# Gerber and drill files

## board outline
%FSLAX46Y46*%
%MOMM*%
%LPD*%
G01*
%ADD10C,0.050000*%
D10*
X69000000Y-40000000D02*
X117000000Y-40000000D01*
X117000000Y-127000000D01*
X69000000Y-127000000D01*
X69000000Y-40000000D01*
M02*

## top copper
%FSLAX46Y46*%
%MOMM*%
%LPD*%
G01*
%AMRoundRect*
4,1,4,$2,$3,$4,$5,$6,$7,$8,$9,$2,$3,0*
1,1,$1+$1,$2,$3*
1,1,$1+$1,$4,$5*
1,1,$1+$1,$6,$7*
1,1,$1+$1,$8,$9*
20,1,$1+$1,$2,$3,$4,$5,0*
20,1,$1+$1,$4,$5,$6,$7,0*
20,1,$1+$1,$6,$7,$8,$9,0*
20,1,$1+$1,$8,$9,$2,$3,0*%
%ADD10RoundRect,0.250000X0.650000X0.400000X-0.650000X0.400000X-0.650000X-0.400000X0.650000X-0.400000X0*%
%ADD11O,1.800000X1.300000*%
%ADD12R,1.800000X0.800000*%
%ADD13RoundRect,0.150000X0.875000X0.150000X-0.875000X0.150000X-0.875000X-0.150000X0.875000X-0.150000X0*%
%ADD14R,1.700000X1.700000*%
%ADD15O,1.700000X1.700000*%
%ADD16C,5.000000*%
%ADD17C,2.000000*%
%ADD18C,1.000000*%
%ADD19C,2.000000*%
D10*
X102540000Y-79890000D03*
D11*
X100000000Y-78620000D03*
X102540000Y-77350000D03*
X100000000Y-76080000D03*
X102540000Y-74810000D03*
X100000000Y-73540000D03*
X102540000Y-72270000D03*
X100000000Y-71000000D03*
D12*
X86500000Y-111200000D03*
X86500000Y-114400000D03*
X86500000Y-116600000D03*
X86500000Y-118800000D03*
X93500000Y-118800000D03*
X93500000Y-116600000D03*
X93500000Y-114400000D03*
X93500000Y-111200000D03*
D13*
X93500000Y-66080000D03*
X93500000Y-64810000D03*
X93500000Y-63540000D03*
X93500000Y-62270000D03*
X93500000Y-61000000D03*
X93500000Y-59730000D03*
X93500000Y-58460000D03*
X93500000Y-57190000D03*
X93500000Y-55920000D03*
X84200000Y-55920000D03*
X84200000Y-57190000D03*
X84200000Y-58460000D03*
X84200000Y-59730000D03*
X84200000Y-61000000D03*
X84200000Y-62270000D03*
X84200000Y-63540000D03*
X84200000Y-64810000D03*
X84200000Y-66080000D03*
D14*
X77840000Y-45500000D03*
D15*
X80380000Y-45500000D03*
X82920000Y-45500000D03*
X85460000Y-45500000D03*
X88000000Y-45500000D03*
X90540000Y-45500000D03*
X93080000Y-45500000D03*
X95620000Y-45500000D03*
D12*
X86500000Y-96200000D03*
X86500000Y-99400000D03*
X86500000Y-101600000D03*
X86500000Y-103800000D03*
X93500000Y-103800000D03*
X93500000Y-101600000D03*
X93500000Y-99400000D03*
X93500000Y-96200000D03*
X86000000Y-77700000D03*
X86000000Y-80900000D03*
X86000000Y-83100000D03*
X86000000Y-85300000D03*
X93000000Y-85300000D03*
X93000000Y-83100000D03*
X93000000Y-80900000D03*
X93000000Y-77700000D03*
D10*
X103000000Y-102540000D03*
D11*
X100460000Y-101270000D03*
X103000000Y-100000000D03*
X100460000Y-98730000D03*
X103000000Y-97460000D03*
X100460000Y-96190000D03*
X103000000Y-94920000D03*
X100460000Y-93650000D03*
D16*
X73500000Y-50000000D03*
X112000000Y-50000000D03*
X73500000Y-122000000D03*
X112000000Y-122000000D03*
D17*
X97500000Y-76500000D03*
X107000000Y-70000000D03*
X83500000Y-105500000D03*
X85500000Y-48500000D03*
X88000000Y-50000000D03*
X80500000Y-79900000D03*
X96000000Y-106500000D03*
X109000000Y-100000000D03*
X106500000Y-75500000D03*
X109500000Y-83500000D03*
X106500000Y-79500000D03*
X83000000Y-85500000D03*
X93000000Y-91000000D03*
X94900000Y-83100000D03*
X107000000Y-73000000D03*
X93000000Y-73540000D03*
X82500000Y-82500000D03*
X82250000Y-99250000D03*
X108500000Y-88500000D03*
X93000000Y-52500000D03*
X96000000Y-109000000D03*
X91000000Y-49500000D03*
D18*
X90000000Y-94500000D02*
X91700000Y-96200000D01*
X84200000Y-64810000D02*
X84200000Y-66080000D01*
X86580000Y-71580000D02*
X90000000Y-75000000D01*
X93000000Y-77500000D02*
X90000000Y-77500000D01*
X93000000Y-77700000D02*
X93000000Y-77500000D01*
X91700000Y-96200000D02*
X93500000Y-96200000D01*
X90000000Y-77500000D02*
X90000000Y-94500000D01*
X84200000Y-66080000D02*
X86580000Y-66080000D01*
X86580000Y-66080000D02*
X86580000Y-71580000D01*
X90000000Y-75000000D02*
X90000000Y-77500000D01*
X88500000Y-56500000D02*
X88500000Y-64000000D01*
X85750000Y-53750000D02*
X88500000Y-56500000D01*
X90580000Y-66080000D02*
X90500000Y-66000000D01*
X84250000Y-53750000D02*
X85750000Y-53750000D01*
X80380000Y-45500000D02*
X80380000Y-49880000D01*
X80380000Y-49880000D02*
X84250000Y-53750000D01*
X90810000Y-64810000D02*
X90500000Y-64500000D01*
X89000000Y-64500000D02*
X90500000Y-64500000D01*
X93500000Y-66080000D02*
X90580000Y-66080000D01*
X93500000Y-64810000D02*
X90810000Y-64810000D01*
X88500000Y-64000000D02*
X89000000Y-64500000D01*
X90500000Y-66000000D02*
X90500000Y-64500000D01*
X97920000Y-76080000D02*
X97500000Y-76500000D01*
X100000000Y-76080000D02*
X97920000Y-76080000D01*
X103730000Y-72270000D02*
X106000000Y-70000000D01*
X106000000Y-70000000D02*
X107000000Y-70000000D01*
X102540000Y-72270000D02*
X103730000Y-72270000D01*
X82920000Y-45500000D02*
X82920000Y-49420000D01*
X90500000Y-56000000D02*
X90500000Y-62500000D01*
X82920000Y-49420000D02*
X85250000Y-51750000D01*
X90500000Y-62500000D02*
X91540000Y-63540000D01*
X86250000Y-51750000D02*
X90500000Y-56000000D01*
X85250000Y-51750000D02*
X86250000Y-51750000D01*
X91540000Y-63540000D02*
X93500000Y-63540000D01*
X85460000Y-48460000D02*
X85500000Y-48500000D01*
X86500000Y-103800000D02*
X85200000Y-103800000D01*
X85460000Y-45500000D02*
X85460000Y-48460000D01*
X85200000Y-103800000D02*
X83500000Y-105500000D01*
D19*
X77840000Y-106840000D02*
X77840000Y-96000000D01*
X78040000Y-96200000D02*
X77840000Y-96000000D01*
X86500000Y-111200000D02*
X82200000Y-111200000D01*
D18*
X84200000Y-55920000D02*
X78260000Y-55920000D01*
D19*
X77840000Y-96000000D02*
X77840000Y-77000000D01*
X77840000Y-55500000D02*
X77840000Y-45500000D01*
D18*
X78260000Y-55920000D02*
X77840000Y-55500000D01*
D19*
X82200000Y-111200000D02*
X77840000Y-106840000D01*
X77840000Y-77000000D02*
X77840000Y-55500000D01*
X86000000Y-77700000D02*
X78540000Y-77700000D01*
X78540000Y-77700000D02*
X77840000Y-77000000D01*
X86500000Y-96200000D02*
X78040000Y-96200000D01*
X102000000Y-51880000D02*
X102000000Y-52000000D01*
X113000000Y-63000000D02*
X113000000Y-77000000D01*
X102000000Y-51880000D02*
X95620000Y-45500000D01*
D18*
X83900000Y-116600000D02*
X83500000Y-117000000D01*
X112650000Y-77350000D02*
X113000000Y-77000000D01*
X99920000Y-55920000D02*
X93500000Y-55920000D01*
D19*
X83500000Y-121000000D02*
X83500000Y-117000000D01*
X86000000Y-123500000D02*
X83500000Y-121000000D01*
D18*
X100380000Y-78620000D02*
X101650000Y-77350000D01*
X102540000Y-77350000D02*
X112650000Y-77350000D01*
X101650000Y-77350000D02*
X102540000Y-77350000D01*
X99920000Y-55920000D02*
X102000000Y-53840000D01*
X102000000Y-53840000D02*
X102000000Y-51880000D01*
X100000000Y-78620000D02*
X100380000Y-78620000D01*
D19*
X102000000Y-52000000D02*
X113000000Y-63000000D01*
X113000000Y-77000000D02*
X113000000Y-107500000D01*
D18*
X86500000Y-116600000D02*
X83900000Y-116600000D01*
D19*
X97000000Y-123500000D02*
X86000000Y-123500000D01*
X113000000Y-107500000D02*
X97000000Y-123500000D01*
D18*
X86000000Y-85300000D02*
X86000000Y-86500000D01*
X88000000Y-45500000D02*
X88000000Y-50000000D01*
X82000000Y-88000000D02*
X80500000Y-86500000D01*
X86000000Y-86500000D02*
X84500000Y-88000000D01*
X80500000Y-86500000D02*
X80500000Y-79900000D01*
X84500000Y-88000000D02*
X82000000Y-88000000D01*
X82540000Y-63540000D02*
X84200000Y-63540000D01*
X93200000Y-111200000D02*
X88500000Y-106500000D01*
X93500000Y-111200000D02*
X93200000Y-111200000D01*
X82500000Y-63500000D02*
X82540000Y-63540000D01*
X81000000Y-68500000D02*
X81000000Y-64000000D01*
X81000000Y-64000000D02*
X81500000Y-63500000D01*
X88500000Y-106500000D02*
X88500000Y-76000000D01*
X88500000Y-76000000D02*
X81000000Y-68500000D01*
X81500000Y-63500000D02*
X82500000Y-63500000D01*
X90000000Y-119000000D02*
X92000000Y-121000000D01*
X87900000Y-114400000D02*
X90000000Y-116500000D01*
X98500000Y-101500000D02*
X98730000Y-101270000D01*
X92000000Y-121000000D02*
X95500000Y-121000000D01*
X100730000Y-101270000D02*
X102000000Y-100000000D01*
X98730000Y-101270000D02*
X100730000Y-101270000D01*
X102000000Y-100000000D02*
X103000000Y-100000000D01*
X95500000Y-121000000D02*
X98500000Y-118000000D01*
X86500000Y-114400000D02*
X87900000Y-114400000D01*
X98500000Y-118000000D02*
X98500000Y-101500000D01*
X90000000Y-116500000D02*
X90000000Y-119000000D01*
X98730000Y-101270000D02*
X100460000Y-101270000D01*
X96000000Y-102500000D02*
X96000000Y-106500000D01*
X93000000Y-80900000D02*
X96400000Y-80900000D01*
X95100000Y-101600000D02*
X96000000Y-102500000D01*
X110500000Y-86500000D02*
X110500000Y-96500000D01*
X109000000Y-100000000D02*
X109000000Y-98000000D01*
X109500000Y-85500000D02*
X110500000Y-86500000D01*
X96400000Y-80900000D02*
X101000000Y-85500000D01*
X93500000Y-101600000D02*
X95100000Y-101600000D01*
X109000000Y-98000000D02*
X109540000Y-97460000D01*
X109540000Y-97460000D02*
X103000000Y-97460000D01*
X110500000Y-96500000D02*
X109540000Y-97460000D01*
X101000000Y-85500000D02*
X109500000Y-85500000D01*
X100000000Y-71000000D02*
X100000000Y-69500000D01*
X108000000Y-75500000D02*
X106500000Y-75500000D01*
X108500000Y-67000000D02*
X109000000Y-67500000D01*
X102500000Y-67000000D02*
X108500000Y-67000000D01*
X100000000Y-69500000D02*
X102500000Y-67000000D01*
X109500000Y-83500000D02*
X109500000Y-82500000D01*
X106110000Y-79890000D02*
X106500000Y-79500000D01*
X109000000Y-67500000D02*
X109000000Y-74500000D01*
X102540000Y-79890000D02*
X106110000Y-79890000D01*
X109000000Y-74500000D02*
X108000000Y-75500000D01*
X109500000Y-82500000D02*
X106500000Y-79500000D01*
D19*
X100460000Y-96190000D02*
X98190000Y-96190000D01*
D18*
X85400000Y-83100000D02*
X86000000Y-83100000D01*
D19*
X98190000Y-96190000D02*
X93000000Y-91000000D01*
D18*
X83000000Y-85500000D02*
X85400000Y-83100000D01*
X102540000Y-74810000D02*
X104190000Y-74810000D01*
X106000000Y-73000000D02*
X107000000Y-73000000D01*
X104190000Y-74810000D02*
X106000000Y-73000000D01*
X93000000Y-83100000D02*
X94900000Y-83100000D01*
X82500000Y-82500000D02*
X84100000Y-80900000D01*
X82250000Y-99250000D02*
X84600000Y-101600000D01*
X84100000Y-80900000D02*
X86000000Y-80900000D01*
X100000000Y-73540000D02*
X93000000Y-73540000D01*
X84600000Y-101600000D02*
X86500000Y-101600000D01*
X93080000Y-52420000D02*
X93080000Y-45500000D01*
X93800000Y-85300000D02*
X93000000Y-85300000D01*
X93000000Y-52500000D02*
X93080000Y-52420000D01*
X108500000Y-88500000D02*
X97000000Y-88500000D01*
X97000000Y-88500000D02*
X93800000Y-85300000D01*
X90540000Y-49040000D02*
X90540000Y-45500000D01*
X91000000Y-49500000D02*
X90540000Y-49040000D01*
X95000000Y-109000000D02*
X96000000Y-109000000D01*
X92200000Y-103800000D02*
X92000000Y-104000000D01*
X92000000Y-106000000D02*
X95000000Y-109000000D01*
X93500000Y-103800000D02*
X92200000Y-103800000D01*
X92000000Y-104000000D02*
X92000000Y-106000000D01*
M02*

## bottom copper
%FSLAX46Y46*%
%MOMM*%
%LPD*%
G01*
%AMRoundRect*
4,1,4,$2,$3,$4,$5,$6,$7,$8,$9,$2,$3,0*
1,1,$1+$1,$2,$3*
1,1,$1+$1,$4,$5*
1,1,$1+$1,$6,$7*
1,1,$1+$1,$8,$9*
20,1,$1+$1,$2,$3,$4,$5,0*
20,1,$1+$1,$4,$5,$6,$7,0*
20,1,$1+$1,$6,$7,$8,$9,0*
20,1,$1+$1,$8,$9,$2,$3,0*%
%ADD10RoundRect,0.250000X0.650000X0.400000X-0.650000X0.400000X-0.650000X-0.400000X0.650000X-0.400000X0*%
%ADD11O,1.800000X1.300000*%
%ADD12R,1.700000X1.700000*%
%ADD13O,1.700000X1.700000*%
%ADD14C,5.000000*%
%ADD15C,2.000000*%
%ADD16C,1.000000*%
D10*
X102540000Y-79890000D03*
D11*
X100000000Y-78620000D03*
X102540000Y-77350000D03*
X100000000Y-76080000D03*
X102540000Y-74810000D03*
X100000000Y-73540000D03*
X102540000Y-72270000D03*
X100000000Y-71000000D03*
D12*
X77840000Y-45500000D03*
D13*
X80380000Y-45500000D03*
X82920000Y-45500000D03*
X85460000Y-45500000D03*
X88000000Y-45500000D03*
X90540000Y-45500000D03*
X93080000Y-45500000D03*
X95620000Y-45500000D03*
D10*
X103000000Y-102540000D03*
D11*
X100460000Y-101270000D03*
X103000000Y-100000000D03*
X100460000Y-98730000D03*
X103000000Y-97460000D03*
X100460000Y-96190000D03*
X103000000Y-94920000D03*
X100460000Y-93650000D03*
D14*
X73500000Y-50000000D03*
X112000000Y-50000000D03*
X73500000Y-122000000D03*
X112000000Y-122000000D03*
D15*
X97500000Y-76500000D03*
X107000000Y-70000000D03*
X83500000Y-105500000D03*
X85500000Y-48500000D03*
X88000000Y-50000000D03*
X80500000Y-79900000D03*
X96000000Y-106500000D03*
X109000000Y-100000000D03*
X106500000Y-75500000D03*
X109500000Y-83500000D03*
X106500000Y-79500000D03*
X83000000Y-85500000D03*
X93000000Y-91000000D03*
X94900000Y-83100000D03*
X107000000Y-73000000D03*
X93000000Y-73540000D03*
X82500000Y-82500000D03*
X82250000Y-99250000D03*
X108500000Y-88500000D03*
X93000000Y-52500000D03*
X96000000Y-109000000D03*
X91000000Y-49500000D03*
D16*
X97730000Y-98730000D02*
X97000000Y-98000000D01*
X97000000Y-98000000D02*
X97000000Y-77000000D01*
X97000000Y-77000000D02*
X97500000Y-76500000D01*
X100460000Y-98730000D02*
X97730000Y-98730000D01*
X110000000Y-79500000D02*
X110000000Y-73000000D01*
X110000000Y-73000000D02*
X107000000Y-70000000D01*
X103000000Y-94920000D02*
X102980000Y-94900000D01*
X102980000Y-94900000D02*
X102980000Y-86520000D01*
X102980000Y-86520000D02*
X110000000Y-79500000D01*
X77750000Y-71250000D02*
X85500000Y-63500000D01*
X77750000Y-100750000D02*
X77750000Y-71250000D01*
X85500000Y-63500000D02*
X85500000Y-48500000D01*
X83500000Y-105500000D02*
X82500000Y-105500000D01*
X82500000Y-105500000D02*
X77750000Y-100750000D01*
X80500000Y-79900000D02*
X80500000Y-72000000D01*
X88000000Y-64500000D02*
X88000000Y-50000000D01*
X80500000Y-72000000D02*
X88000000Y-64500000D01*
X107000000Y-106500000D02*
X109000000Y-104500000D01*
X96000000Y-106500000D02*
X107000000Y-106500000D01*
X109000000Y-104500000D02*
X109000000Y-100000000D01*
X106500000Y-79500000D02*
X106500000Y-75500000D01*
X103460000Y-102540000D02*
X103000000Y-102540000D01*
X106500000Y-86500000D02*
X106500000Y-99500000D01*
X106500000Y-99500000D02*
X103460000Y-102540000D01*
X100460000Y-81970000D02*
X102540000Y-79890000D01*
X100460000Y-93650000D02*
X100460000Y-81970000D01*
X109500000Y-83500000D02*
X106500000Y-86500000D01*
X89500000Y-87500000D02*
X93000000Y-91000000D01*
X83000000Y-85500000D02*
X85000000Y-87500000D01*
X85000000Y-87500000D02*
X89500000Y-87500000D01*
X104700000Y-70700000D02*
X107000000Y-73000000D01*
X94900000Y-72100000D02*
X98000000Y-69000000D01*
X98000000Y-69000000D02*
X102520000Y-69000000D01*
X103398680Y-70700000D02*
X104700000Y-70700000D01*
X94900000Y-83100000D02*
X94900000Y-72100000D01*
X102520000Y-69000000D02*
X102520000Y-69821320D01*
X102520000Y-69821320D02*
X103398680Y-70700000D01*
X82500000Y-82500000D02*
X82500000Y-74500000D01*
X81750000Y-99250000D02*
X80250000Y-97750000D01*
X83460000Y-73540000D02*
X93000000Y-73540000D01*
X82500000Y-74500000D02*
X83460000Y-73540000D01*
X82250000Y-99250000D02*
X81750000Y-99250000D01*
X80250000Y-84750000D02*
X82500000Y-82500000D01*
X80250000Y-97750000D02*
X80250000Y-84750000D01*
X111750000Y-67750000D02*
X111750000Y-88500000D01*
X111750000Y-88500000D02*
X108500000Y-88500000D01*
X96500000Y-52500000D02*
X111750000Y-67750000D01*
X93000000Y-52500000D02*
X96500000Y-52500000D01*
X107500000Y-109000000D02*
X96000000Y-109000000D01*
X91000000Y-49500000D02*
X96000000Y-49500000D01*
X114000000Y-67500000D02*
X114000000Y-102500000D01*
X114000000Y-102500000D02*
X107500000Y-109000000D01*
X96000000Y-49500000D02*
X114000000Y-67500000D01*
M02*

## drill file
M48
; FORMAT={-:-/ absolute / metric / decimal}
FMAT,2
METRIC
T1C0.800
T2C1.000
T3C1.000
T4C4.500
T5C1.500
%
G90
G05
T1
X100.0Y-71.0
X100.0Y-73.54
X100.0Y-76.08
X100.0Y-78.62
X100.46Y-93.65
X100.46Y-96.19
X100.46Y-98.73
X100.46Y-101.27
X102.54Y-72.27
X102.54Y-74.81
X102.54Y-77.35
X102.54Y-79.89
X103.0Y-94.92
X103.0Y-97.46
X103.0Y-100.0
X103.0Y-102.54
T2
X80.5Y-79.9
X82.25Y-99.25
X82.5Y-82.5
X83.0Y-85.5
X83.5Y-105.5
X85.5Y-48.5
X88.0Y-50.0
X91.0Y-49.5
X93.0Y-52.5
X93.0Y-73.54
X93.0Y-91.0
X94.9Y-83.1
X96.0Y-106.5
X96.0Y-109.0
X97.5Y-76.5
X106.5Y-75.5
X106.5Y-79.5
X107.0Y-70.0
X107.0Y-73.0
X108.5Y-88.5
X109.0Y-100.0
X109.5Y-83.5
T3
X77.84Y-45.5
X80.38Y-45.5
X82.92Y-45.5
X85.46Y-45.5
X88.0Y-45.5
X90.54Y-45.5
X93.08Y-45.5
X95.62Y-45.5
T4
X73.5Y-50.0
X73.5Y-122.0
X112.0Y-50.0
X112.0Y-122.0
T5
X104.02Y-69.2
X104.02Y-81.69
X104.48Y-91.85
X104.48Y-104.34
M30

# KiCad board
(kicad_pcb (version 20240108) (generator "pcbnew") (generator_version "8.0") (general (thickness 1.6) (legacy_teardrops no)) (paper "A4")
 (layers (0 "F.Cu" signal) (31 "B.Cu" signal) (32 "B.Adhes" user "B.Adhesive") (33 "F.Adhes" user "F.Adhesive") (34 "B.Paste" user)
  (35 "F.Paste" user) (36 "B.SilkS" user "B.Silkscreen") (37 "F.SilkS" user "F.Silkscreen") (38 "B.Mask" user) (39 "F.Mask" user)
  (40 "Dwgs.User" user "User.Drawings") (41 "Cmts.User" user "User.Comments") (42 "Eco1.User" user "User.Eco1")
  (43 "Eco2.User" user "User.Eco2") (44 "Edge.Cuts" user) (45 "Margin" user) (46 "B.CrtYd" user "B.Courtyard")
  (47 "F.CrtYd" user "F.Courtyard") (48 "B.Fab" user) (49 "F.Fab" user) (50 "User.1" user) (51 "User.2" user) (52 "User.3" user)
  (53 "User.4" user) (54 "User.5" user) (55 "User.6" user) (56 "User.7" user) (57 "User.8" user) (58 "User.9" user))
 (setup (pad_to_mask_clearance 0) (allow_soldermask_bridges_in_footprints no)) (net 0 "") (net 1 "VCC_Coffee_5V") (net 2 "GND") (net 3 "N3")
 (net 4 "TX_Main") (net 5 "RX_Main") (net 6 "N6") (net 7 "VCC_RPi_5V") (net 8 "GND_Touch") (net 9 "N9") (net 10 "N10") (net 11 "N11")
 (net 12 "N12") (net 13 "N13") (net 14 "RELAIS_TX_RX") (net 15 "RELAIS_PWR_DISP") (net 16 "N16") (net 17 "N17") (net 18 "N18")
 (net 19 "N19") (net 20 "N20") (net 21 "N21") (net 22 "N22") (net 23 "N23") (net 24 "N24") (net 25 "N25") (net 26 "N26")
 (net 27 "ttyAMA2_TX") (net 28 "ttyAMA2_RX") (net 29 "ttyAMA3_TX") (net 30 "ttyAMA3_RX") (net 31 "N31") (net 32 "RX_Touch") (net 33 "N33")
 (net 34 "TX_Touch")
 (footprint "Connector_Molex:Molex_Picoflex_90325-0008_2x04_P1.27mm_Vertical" (layer "F.Cu") (at 102.54 79.89 180)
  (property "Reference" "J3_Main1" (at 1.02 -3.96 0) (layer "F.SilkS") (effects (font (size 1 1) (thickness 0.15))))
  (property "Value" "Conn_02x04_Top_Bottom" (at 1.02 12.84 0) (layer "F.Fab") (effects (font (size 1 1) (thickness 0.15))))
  (pad "" np_thru_hole circle (at -1.48 -1.8 180) (size 1.5 1.5) (drill 1.5) (layers "*.Cu" "*.Mask"))
  (pad "" np_thru_hole circle (at -1.48 10.69 180) (size 1.5 1.5) (drill 1.5) (layers "*.Cu" "*.Mask"))
  (pad "1" thru_hole roundrect (at 0 0 180) (size 1.8 1.3) (drill 0.8) (layers "*.Cu" "*.Mask") (remove_unused_layers no)
   (roundrect_rratio 0.192308) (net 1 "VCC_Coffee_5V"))
  (pad "2" thru_hole oval (at 2.54 1.27 180) (size 1.8 1.3) (drill 0.8) (layers "*.Cu" "*.Mask") (remove_unused_layers no) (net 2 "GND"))
  (pad "3" thru_hole oval (at 0 2.54 180) (size 1.8 1.3) (drill 0.8) (layers "*.Cu" "*.Mask") (remove_unused_layers no) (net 2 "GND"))
  (pad "4" thru_hole oval (at 2.54 3.81 180) (size 1.8 1.3) (drill 0.8) (layers "*.Cu" "*.Mask") (remove_unused_layers no) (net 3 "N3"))
  (pad "5" thru_hole oval (at 0 5.08 180) (size 1.8 1.3) (drill 0.8) (layers "*.Cu" "*.Mask") (remove_unused_layers no) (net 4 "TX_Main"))
  (pad "6" thru_hole oval (at 2.54 6.35 180) (size 1.8 1.3) (drill 0.8) (layers "*.Cu" "*.Mask") (remove_unused_layers no) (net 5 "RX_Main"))
  (pad "7" thru_hole oval (at 0 7.62 180) (size 1.8 1.3) (drill 0.8) (layers "*.Cu" "*.Mask") (remove_unused_layers no) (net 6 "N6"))
  (pad "8" thru_hole oval (at 2.54 8.89 180) (size 1.8 1.3) (drill 0.8) (layers "*.Cu" "*.Mask") (remove_unused_layers no)
   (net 1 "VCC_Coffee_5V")))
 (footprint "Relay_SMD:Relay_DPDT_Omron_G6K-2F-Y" (layer "F.Cu") (at 90 115)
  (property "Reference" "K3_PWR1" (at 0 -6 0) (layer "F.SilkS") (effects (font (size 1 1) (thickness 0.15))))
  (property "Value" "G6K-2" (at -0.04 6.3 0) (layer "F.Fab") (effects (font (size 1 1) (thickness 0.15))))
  (pad "1" smd rect (at -3.5 -3.8) (size 1.8 0.8) (layers "F.Cu" "F.Paste" "F.Mask") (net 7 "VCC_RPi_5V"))
  (pad "2" smd rect (at -3.5 -0.6) (size 1.8 0.8) (layers "F.Cu" "F.Paste" "F.Mask") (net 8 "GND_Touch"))
  (pad "3" smd rect (at -3.5 1.6) (size 1.8 0.8) (layers "F.Cu" "F.Paste" "F.Mask") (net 2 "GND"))
  (pad "4" smd rect (at -3.5 3.8) (size 1.8 0.8) (layers "F.Cu" "F.Paste" "F.Mask") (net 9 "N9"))
  (pad "5" smd rect (at 3.5 3.8) (size 1.8 0.8) (layers "F.Cu" "F.Paste" "F.Mask") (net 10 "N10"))
  (pad "6" smd rect (at 3.5 1.6) (size 1.8 0.8) (layers "F.Cu" "F.Paste" "F.Mask") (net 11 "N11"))
  (pad "7" smd rect (at 3.5 -0.6) (size 1.8 0.8) (layers "F.Cu" "F.Paste" "F.Mask") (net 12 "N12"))
  (pad "8" smd rect (at 3.5 -3.8) (size 1.8 0.8) (layers "F.Cu" "F.Paste" "F.Mask") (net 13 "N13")))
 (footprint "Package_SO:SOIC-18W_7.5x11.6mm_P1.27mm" (layer "F.Cu") (at 88.85 61 180)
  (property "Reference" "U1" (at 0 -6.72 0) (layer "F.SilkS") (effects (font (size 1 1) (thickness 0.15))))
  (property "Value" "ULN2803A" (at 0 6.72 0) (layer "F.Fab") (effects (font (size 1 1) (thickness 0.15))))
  (pad "1" smd roundrect (at -4.65 -5.08 180) (size 2.05 0.6) (layers "F.Cu" "F.Paste" "F.Mask") (roundrect_rratio 0.25)
   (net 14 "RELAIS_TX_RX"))
  (pad "2" smd roundrect (at -4.65 -3.81 180) (size 2.05 0.6) (layers "F.Cu" "F.Paste" "F.Mask") (roundrect_rratio 0.25)
   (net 14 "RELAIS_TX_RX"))
  (pad "3" smd roundrect (at -4.65 -2.54 180) (size 2.05 0.6) (layers "F.Cu" "F.Paste" "F.Mask") (roundrect_rratio 0.25)
   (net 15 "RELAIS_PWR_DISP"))
  (pad "4" smd roundrect (at -4.65 -1.27 180) (size 2.05 0.6) (layers "F.Cu" "F.Paste" "F.Mask") (roundrect_rratio 0.25) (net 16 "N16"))
  (pad "5" smd roundrect (at -4.65 0 180) (size 2.05 0.6) (layers "F.Cu" "F.Paste" "F.Mask") (roundrect_rratio 0.25) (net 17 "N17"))
  (pad "6" smd roundrect (at -4.65 1.27 180) (size 2.05 0.6) (layers "F.Cu" "F.Paste" "F.Mask") (roundrect_rratio 0.25) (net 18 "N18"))
  (pad "7" smd roundrect (at -4.65 2.54 180) (size 2.05 0.6) (layers "F.Cu" "F.Paste" "F.Mask") (roundrect_rratio 0.25) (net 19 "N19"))
  (pad "8" smd roundrect (at -4.65 3.81 180) (size 2.05 0.6) (layers "F.Cu" "F.Paste" "F.Mask") (roundrect_rratio 0.25) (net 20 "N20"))
  (pad "9" smd roundrect (at -4.65 5.08 180) (size 2.05 0.6) (layers "F.Cu" "F.Paste" "F.Mask") (roundrect_rratio 0.25) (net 2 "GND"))
  (pad "10" smd roundrect (at 4.65 5.08 180) (size 2.05 0.6) (layers "F.Cu" "F.Paste" "F.Mask") (roundrect_rratio 0.25) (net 7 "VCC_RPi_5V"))
  (pad "11" smd roundrect (at 4.65 3.81 180) (size 2.05 0.6) (layers "F.Cu" "F.Paste" "F.Mask") (roundrect_rratio 0.25) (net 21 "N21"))
  (pad "12" smd roundrect (at 4.65 2.54 180) (size 2.05 0.6) (layers "F.Cu" "F.Paste" "F.Mask") (roundrect_rratio 0.25) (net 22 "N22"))
  (pad "13" smd roundrect (at 4.65 1.27 180) (size 2.05 0.6) (layers "F.Cu" "F.Paste" "F.Mask") (roundrect_rratio 0.25) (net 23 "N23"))
  (pad "14" smd roundrect (at 4.65 0 180) (size 2.05 0.6) (layers "F.Cu" "F.Paste" "F.Mask") (roundrect_rratio 0.25) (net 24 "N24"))
  (pad "15" smd roundrect (at 4.65 -1.27 180) (size 2.05 0.6) (layers "F.Cu" "F.Paste" "F.Mask") (roundrect_rratio 0.25) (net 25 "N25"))
  (pad "16" smd roundrect (at 4.65 -2.54 180) (size 2.05 0.6) (layers "F.Cu" "F.Paste" "F.Mask") (roundrect_rratio 0.25) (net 13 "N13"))
  (pad "17" smd roundrect (at 4.65 -3.81 180) (size 2.05 0.6) (layers "F.Cu" "F.Paste" "F.Mask") (roundrect_rratio 0.25) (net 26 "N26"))
  (pad "18" smd roundrect (at 4.65 -5.08 180) (size 2.05 0.6) (layers "F.Cu" "F.Paste" "F.Mask") (roundrect_rratio 0.25) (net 26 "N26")))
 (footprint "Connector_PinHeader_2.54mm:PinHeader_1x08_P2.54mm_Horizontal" (layer "F.Cu") (at 77.84 45.5 90)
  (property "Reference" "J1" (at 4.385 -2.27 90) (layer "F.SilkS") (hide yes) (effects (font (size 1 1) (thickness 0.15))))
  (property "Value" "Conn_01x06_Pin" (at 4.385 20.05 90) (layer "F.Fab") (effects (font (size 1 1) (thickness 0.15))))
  (pad "1" thru_hole rect (at 0 0 90) (size 1.7 1.7) (drill 1) (layers "*.Cu" "*.Mask") (remove_unused_layers no) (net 7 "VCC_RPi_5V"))
  (pad "2" thru_hole oval (at 0 2.54 90) (size 1.7 1.7) (drill 1) (layers "*.Cu" "*.Mask") (remove_unused_layers no) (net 14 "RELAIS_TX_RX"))
  (pad "3" thru_hole oval (at 0 5.08 90) (size 1.7 1.7) (drill 1) (layers "*.Cu" "*.Mask") (remove_unused_layers no)
   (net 15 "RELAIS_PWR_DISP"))
  (pad "4" thru_hole oval (at 0 7.62 90) (size 1.7 1.7) (drill 1) (layers "*.Cu" "*.Mask") (remove_unused_layers no) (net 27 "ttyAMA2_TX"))
  (pad "5" thru_hole oval (at 0 10.16 90) (size 1.7 1.7) (drill 1) (layers "*.Cu" "*.Mask") (remove_unused_layers no) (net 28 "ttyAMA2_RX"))
  (pad "6" thru_hole oval (at 0 12.7 90) (size 1.7 1.7) (drill 1) (layers "*.Cu" "*.Mask") (remove_unused_layers no) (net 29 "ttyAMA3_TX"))
  (pad "7" thru_hole oval (at 0 15.24 90) (size 1.7 1.7) (drill 1) (layers "*.Cu" "*.Mask") (remove_unused_layers no) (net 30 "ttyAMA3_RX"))
  (pad "8" thru_hole oval (at 0 17.78 90) (size 1.7 1.7) (drill 1) (layers "*.Cu" "*.Mask") (remove_unused_layers no) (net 2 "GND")))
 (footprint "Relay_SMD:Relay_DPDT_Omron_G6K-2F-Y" (layer "F.Cu") (at 90 100)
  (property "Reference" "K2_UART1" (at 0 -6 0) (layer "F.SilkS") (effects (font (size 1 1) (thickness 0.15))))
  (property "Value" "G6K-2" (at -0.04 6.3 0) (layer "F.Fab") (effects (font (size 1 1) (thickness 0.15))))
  (pad "1" smd rect (at -3.5 -3.8) (size 1.8 0.8) (layers "F.Cu" "F.Paste" "F.Mask") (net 7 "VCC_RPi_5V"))
  (pad "2" smd rect (at -3.5 -0.6) (size 1.8 0.8) (layers "F.Cu" "F.Paste" "F.Mask") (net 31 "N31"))
  (pad "3" smd rect (at -3.5 1.6) (size 1.8 0.8) (layers "F.Cu" "F.Paste" "F.Mask") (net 5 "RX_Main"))
  (pad "4" smd rect (at -3.5 3.8) (size 1.8 0.8) (layers "F.Cu" "F.Paste" "F.Mask") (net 27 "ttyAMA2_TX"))
  (pad "5" smd rect (at 3.5 3.8) (size 1.8 0.8) (layers "F.Cu" "F.Paste" "F.Mask") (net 29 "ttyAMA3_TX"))
  (pad "6" smd rect (at 3.5 1.6) (size 1.8 0.8) (layers "F.Cu" "F.Paste" "F.Mask") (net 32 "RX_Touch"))
  (pad "7" smd rect (at 3.5 -0.6) (size 1.8 0.8) (layers "F.Cu" "F.Paste" "F.Mask") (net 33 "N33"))
  (pad "8" smd rect (at 3.5 -3.8) (size 1.8 0.8) (layers "F.Cu" "F.Paste" "F.Mask") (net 26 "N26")))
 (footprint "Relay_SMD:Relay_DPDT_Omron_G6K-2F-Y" (layer "F.Cu") (at 89.5 81.5)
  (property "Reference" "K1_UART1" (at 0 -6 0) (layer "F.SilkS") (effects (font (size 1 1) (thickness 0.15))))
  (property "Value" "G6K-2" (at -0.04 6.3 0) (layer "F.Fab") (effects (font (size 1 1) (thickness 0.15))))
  (pad "1" smd rect (at -3.5 -3.8) (size 1.8 0.8) (layers "F.Cu" "F.Paste" "F.Mask") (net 7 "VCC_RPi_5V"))
  (pad "2" smd rect (at -3.5 -0.6) (size 1.8 0.8) (layers "F.Cu" "F.Paste" "F.Mask") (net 5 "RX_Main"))
  (pad "3" smd rect (at -3.5 1.6) (size 1.8 0.8) (layers "F.Cu" "F.Paste" "F.Mask") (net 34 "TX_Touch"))
  (pad "4" smd rect (at -3.5 3.8) (size 1.8 0.8) (layers "F.Cu" "F.Paste" "F.Mask") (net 28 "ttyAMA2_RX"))
  (pad "5" smd rect (at 3.5 3.8) (size 1.8 0.8) (layers "F.Cu" "F.Paste" "F.Mask") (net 30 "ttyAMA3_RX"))
  (pad "6" smd rect (at 3.5 1.6) (size 1.8 0.8) (layers "F.Cu" "F.Paste" "F.Mask") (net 4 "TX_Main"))
  (pad "7" smd rect (at 3.5 -0.6) (size 1.8 0.8) (layers "F.Cu" "F.Paste" "F.Mask") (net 32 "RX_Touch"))
  (pad "8" smd rect (at 3.5 -3.8) (size 1.8 0.8) (layers "F.Cu" "F.Paste" "F.Mask") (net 26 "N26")))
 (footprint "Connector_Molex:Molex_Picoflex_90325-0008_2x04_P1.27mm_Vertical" (layer "F.Cu") (at 103 102.54 180)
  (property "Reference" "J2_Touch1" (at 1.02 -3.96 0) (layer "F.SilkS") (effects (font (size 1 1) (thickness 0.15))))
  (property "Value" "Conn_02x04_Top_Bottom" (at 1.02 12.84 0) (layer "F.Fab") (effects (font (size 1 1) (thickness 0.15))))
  (pad "" np_thru_hole circle (at -1.48 -1.8 180) (size 1.5 1.5) (drill 1.5) (layers "*.Cu" "*.Mask"))
  (pad "" np_thru_hole circle (at -1.48 10.69 180) (size 1.5 1.5) (drill 1.5) (layers "*.Cu" "*.Mask"))
  (pad "1" thru_hole roundrect (at 0 0 180) (size 1.8 1.3) (drill 0.8) (layers "*.Cu" "*.Mask") (remove_unused_layers no)
   (roundrect_rratio 0.192308) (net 1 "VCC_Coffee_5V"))
  (pad "2" thru_hole oval (at 2.54 1.27 180) (size 1.8 1.3) (drill 0.8) (layers "*.Cu" "*.Mask") (remove_unused_layers no)
   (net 8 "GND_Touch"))
  (pad "3" thru_hole oval (at 0 2.54 180) (size 1.8 1.3) (drill 0.8) (layers "*.Cu" "*.Mask") (remove_unused_layers no) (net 8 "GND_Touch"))
  (pad "4" thru_hole oval (at 2.54 3.81 180) (size 1.8 1.3) (drill 0.8) (layers "*.Cu" "*.Mask") (remove_unused_layers no) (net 3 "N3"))
  (pad "5" thru_hole oval (at 0 5.08 180) (size 1.8 1.3) (drill 0.8) (layers "*.Cu" "*.Mask") (remove_unused_layers no) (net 32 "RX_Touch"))
  (pad "6" thru_hole oval (at 2.54 6.35 180) (size 1.8 1.3) (drill 0.8) (layers "*.Cu" "*.Mask") (remove_unused_layers no)
   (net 34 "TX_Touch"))
  (pad "7" thru_hole oval (at 0 7.62 180) (size 1.8 1.3) (drill 0.8) (layers "*.Cu" "*.Mask") (remove_unused_layers no) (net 6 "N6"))
  (pad "8" thru_hole oval (at 2.54 8.89 180) (size 1.8 1.3) (drill 0.8) (layers "*.Cu" "*.Mask") (remove_unused_layers no)
   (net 1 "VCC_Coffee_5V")))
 (gr_rect (start 69 40) (end 117 127) (stroke (width 0.05) (type default)) (fill none) (layer "Edge.Cuts"))
 (via (at 73.5 50) (size 5) (drill 4.5) (layers "F.Cu" "B.Cu") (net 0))
 (via (at 112 50) (size 5) (drill 4.5) (layers "F.Cu" "B.Cu") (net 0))
 (via (at 73.5 122) (size 5) (drill 4.5) (layers "F.Cu" "B.Cu") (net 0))
 (via (at 112 122) (size 5) (drill 4.5) (layers "F.Cu" "B.Cu") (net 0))
 (segment (start 90 94.5) (end 91.7 96.2) (width 1) (layer "F.Cu") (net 26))
 (segment (start 84.2 64.81) (end 84.2 66.08) (width 1) (layer "F.Cu") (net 26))
 (segment (start 86.58 71.58) (end 90 75) (width 1) (layer "F.Cu") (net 26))
 (segment (start 93 77.5) (end 90 77.5) (width 1) (layer "F.Cu") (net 26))
 (segment (start 93 77.7) (end 93 77.5) (width 1) (layer "F.Cu") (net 26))
 (segment (start 91.7 96.2) (end 93.5 96.2) (width 1) (layer "F.Cu") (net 26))
 (segment (start 90 77.5) (end 90 94.5) (width 1) (layer "F.Cu") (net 26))
 (segment (start 84.2 66.08) (end 86.58 66.08) (width 1) (layer "F.Cu") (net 26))
 (segment (start 86.58 66.08) (end 86.58 71.58) (width 1) (layer "F.Cu") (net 26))
 (segment (start 90 75) (end 90 77.5) (width 1) (layer "F.Cu") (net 26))
 (segment (start 88.5 56.5) (end 88.5 64) (width 1) (layer "F.Cu") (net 14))
 (segment (start 85.75 53.75) (end 88.5 56.5) (width 1) (layer "F.Cu") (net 14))
 (segment (start 90.58 66.08) (end 90.5 66) (width 1) (layer "F.Cu") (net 14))
 (segment (start 84.25 53.75) (end 85.75 53.75) (width 1) (layer "F.Cu") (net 14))
 (segment (start 80.38 45.5) (end 80.38 49.88) (width 1) (layer "F.Cu") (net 14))
 (segment (start 80.38 49.88) (end 84.25 53.75) (width 1) (layer "F.Cu") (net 14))
 (segment (start 90.81 64.81) (end 90.5 64.5) (width 1) (layer "F.Cu") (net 14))
 (segment (start 89 64.5) (end 90.5 64.5) (width 1) (layer "F.Cu") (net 14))
 (segment (start 93.5 66.08) (end 90.58 66.08) (width 1) (layer "F.Cu") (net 14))
 (segment (start 93.5 64.81) (end 90.81 64.81) (width 1) (layer "F.Cu") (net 14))
 (segment (start 88.5 64) (end 89 64.5) (width 1) (layer "F.Cu") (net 14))
 (segment (start 90.5 66) (end 90.5 64.5) (width 1) (layer "F.Cu") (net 14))
 (segment (start 97.92 76.08) (end 97.5 76.5) (width 1) (layer "F.Cu") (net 3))
 (segment (start 100 76.08) (end 97.92 76.08) (width 1) (layer "F.Cu") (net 3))
 (via (at 97.5 76.5) (size 2) (drill 1) (layers "F.Cu" "B.Cu") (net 3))
 (segment (start 97.73 98.73) (end 97 98) (width 1) (layer "B.Cu") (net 3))
 (segment (start 97 98) (end 97 77) (width 1) (layer "B.Cu") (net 3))
 (segment (start 97 77) (end 97.5 76.5) (width 1) (layer "B.Cu") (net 3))
 (segment (start 100.46 98.73) (end 97.73 98.73) (width 1) (layer "B.Cu") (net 3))
 (segment (start 103.73 72.27) (end 106 70) (width 1) (layer "F.Cu") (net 6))
 (segment (start 106 70) (end 107 70) (width 1) (layer "F.Cu") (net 6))
 (segment (start 102.54 72.27) (end 103.73 72.27) (width 1) (layer "F.Cu") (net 6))
 (via (at 107 70) (size 2) (drill 1) (layers "F.Cu" "B.Cu") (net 6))
 (segment (start 110 79.5) (end 110 73) (width 1) (layer "B.Cu") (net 6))
 (segment (start 110 73) (end 107 70) (width 1) (layer "B.Cu") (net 6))
 (segment (start 103 94.92) (end 102.98 94.9) (width 1) (layer "B.Cu") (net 6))
 (segment (start 102.98 94.9) (end 102.98 86.52) (width 1) (layer "B.Cu") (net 6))
 (segment (start 102.98 86.52) (end 110 79.5) (width 1) (layer "B.Cu") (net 6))
 (segment (start 82.92 45.5) (end 82.92 49.42) (width 1) (layer "F.Cu") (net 15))
 (segment (start 90.5 56) (end 90.5 62.5) (width 1) (layer "F.Cu") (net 15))
 (segment (start 82.92 49.42) (end 85.25 51.75) (width 1) (layer "F.Cu") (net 15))
 (segment (start 90.5 62.5) (end 91.54 63.54) (width 1) (layer "F.Cu") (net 15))
 (segment (start 86.25 51.75) (end 90.5 56) (width 1) (layer "F.Cu") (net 15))
 (segment (start 85.25 51.75) (end 86.25 51.75) (width 1) (layer "F.Cu") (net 15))
 (segment (start 91.54 63.54) (end 93.5 63.54) (width 1) (layer "F.Cu") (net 15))
 (segment (start 85.46 48.46) (end 85.5 48.5) (width 1) (layer "F.Cu") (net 27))
 (segment (start 86.5 103.8) (end 85.2 103.8) (width 1) (layer "F.Cu") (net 27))
 (segment (start 85.46 45.5) (end 85.46 48.46) (width 1) (layer "F.Cu") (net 27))
 (segment (start 85.2 103.8) (end 83.5 105.5) (width 1) (layer "F.Cu") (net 27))
 (via (at 83.5 105.5) (size 2) (drill 1) (layers "F.Cu" "B.Cu") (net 27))
 (via (at 85.5 48.5) (size 2) (drill 1) (layers "F.Cu" "B.Cu") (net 27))
 (segment (start 77.75 71.25) (end 85.5 63.5) (width 1) (layer "B.Cu") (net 27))
 (segment (start 77.75 100.75) (end 77.75 71.25) (width 1) (layer "B.Cu") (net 27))
 (segment (start 85.5 63.5) (end 85.5 48.5) (width 1) (layer "B.Cu") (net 27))
 (segment (start 83.5 105.5) (end 82.5 105.5) (width 1) (layer "B.Cu") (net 27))
 (segment (start 82.5 105.5) (end 77.75 100.75) (width 1) (layer "B.Cu") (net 27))
 (segment (start 77.84 106.84) (end 77.84 96) (width 2) (layer "F.Cu") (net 7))
 (segment (start 78.04 96.2) (end 77.84 96) (width 2) (layer "F.Cu") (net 7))
 (segment (start 86.5 111.2) (end 82.2 111.2) (width 2) (layer "F.Cu") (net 7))
 (segment (start 84.2 55.92) (end 78.26 55.92) (width 1) (layer "F.Cu") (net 7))
 (segment (start 77.84 96) (end 77.84 77) (width 2) (layer "F.Cu") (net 7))
 (segment (start 77.84 55.5) (end 77.84 45.5) (width 2) (layer "F.Cu") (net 7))
 (segment (start 78.26 55.92) (end 77.84 55.5) (width 1) (layer "F.Cu") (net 7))
 (segment (start 82.2 111.2) (end 77.84 106.84) (width 2) (layer "F.Cu") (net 7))
 (segment (start 77.84 77) (end 77.84 55.5) (width 2) (layer "F.Cu") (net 7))
 (segment (start 86 77.7) (end 78.54 77.7) (width 2) (layer "F.Cu") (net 7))
 (segment (start 78.54 77.7) (end 77.84 77) (width 2) (layer "F.Cu") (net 7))
 (segment (start 86.5 96.2) (end 78.04 96.2) (width 2) (layer "F.Cu") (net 7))
 (segment (start 102 51.88) (end 102 52) (width 2) (layer "F.Cu") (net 2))
 (segment (start 113 63) (end 113 77) (width 2) (layer "F.Cu") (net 2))
 (segment (start 102 51.88) (end 95.62 45.5) (width 2) (layer "F.Cu") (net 2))
 (segment (start 83.9 116.6) (end 83.5 117) (width 1) (layer "F.Cu") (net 2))
 (segment (start 112.65 77.35) (end 113 77) (width 1) (layer "F.Cu") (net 2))
 (segment (start 99.92 55.92) (end 93.5 55.92) (width 1) (layer "F.Cu") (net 2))
 (segment (start 83.5 121) (end 83.5 117) (width 2) (layer "F.Cu") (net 2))
 (segment (start 86 123.5) (end 83.5 121) (width 2) (layer "F.Cu") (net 2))
 (segment (start 100.38 78.62) (end 101.65 77.35) (width 1) (layer "F.Cu") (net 2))
 (segment (start 102.54 77.35) (end 112.65 77.35) (width 1) (layer "F.Cu") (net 2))
 (segment (start 101.65 77.35) (end 102.54 77.35) (width 1) (layer "F.Cu") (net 2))
 (segment (start 99.92 55.92) (end 102 53.84) (width 1) (layer "F.Cu") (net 2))
 (segment (start 102 53.84) (end 102 51.88) (width 1) (layer "F.Cu") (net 2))
 (segment (start 100 78.62) (end 100.38 78.62) (width 1) (layer "F.Cu") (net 2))
 (segment (start 102 52) (end 113 63) (width 2) (layer "F.Cu") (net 2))
 (segment (start 113 77) (end 113 107.5) (width 2) (layer "F.Cu") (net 2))
 (segment (start 86.5 116.6) (end 83.9 116.6) (width 1) (layer "F.Cu") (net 2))
 (segment (start 97 123.5) (end 86 123.5) (width 2) (layer "F.Cu") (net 2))
 (segment (start 113 107.5) (end 97 123.5) (width 2) (layer "F.Cu") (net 2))
 (segment (start 86 85.3) (end 86 86.5) (width 1) (layer "F.Cu") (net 28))
 (segment (start 88 45.5) (end 88 50) (width 1) (layer "F.Cu") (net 28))
 (segment (start 82 88) (end 80.5 86.5) (width 1) (layer "F.Cu") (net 28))
 (segment (start 86 86.5) (end 84.5 88) (width 1) (layer "F.Cu") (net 28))
 (segment (start 80.5 86.5) (end 80.5 79.9) (width 1) (layer "F.Cu") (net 28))
 (segment (start 84.5 88) (end 82 88) (width 1) (layer "F.Cu") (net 28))
 (via (at 88 50) (size 2) (drill 1) (layers "F.Cu" "B.Cu") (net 28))
 (via (at 80.5 79.9) (size 2) (drill 1) (layers "F.Cu" "B.Cu") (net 28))
 (segment (start 80.5 79.9) (end 80.5 72) (width 1) (layer "B.Cu") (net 28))
 (segment (start 88 64.5) (end 88 50) (width 1) (layer "B.Cu") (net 28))
 (segment (start 80.5 72) (end 88 64.5) (width 1) (layer "B.Cu") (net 28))
 (segment (start 82.54 63.54) (end 84.2 63.54) (width 1) (layer "F.Cu") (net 13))
 (segment (start 93.2 111.2) (end 88.5 106.5) (width 1) (layer "F.Cu") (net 13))
 (segment (start 93.5 111.2) (end 93.2 111.2) (width 1) (layer "F.Cu") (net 13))
 (segment (start 82.5 63.5) (end 82.54 63.54) (width 1) (layer "F.Cu") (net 13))
 (segment (start 81 68.5) (end 81 64) (width 1) (layer "F.Cu") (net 13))
 (segment (start 81 64) (end 81.5 63.5) (width 1) (layer "F.Cu") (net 13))
 (segment (start 88.5 106.5) (end 88.5 76) (width 1) (layer "F.Cu") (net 13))
 (segment (start 88.5 76) (end 81 68.5) (width 1) (layer "F.Cu") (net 13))
 (segment (start 81.5 63.5) (end 82.5 63.5) (width 1) (layer "F.Cu") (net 13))
 (segment (start 90 119) (end 92 121) (width 1) (layer "F.Cu") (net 8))
 (segment (start 87.9 114.4) (end 90 116.5) (width 1) (layer "F.Cu") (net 8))
 (segment (start 98.5 101.5) (end 98.73 101.27) (width 1) (layer "F.Cu") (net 8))
 (segment (start 92 121) (end 95.5 121) (width 1) (layer "F.Cu") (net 8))
 (segment (start 100.73 101.27) (end 102 100) (width 1) (layer "F.Cu") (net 8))
 (segment (start 98.73 101.27) (end 100.73 101.27) (width 1) (layer "F.Cu") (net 8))
 (segment (start 102 100) (end 103 100) (width 1) (layer "F.Cu") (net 8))
 (segment (start 95.5 121) (end 98.5 118) (width 1) (layer "F.Cu") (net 8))
 (segment (start 86.5 114.4) (end 87.9 114.4) (width 1) (layer "F.Cu") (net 8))
 (segment (start 98.5 118) (end 98.5 101.5) (width 1) (layer "F.Cu") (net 8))
 (segment (start 90 116.5) (end 90 119) (width 1) (layer "F.Cu") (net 8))
 (segment (start 98.73 101.27) (end 100.46 101.27) (width 1) (layer "F.Cu") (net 8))
 (segment (start 96 102.5) (end 96 106.5) (width 1) (layer "F.Cu") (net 32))
 (segment (start 93 80.9) (end 96.4 80.9) (width 1) (layer "F.Cu") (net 32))
 (segment (start 95.1 101.6) (end 96 102.5) (width 1) (layer "F.Cu") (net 32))
 (segment (start 110.5 86.5) (end 110.5 96.5) (width 1) (layer "F.Cu") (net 32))
 (segment (start 109 100) (end 109 98) (width 1) (layer "F.Cu") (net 32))
 (segment (start 109.5 85.5) (end 110.5 86.5) (width 1) (layer "F.Cu") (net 32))
 (segment (start 96.4 80.9) (end 101 85.5) (width 1) (layer "F.Cu") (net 32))
 (segment (start 93.5 101.6) (end 95.1 101.6) (width 1) (layer "F.Cu") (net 32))
 (segment (start 109 98) (end 109.54 97.46) (width 1) (layer "F.Cu") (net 32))
 (segment (start 109.54 97.46) (end 103 97.46) (width 1) (layer "F.Cu") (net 32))
 (segment (start 110.5 96.5) (end 109.54 97.46) (width 1) (layer "F.Cu") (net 32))
 (segment (start 101 85.5) (end 109.5 85.5) (width 1) (layer "F.Cu") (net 32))
 (via (at 96 106.5) (size 2) (drill 1) (layers "F.Cu" "B.Cu") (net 32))
 (via (at 109 100) (size 2) (drill 1) (layers "F.Cu" "B.Cu") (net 32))
 (segment (start 107 106.5) (end 109 104.5) (width 1) (layer "B.Cu") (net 32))
 (segment (start 96 106.5) (end 107 106.5) (width 1) (layer "B.Cu") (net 32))
 (segment (start 109 104.5) (end 109 100) (width 1) (layer "B.Cu") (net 32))
 (segment (start 100 71) (end 100 69.5) (width 1) (layer "F.Cu") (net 1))
 (segment (start 108 75.5) (end 106.5 75.5) (width 1) (layer "F.Cu") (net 1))
 (segment (start 108.5 67) (end 109 67.5) (width 1) (layer "F.Cu") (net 1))
 (segment (start 102.5 67) (end 108.5 67) (width 1) (layer "F.Cu") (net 1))
 (segment (start 100 69.5) (end 102.5 67) (width 1) (layer "F.Cu") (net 1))
 (segment (start 109.5 83.5) (end 109.5 82.5) (width 1) (layer "F.Cu") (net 1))
 (segment (start 106.11 79.89) (end 106.5 79.5) (width 1) (layer "F.Cu") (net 1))
 (segment (start 109 67.5) (end 109 74.5) (width 1) (layer "F.Cu") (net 1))
 (segment (start 102.54 79.89) (end 106.11 79.89) (width 1) (layer "F.Cu") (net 1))
 (segment (start 109 74.5) (end 108 75.5) (width 1) (layer "F.Cu") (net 1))
 (segment (start 109.5 82.5) (end 106.5 79.5) (width 1) (layer "F.Cu") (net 1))
 (via (at 106.5 75.5) (size 2) (drill 1) (layers "F.Cu" "B.Cu") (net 1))
 (via (at 109.5 83.5) (size 2) (drill 1) (layers "F.Cu" "B.Cu") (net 1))
 (via (at 106.5 79.5) (size 2) (drill 1) (layers "F.Cu" "B.Cu") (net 1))
 (segment (start 106.5 79.5) (end 106.5 75.5) (width 1) (layer "B.Cu") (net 1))
 (segment (start 103.46 102.54) (end 103 102.54) (width 1) (layer "B.Cu") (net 1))
 (segment (start 106.5 86.5) (end 106.5 99.5) (width 1) (layer "B.Cu") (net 1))
 (segment (start 106.5 99.5) (end 103.46 102.54) (width 1) (layer "B.Cu") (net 1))
 (segment (start 100.46 81.97) (end 102.54 79.89) (width 1) (layer "B.Cu") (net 1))
 (segment (start 100.46 93.65) (end 100.46 81.97) (width 1) (layer "B.Cu") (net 1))
 (segment (start 109.5 83.5) (end 106.5 86.5) (width 1) (layer "B.Cu") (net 1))
 (segment (start 100.46 96.19) (end 98.19 96.19) (width 2) (layer "F.Cu") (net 34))
 (segment (start 85.4 83.1) (end 86 83.1) (width 1) (layer "F.Cu") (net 34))
 (segment (start 98.19 96.19) (end 93 91) (width 2) (layer "F.Cu") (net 34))
 (segment (start 83 85.5) (end 85.4 83.1) (width 1) (layer "F.Cu") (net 34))
 (via (at 83 85.5) (size 2) (drill 1) (layers "F.Cu" "B.Cu") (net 34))
 (via (at 93 91) (size 2) (drill 1) (layers "F.Cu" "B.Cu") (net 34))
 (segment (start 89.5 87.5) (end 93 91) (width 1) (layer "B.Cu") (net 34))
 (segment (start 83 85.5) (end 85 87.5) (width 1) (layer "B.Cu") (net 34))
 (segment (start 85 87.5) (end 89.5 87.5) (width 1) (layer "B.Cu") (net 34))
 (segment (start 102.54 74.81) (end 104.19 74.81) (width 1) (layer "F.Cu") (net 4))
 (segment (start 106 73) (end 107 73) (width 1) (layer "F.Cu") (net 4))
 (segment (start 104.19 74.81) (end 106 73) (width 1) (layer "F.Cu") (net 4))
 (segment (start 93 83.1) (end 94.9 83.1) (width 1) (layer "F.Cu") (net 4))
 (via (at 94.9 83.1) (size 2) (drill 1) (layers "F.Cu" "B.Cu") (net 4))
 (via (at 107 73) (size 2) (drill 1) (layers "F.Cu" "B.Cu") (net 4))
 (segment (start 104.7 70.7) (end 107 73) (width 1) (layer "B.Cu") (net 4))
 (segment (start 94.9 72.1) (end 98 69) (width 1) (layer "B.Cu") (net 4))
 (segment (start 98 69) (end 102.52 69) (width 1) (layer "B.Cu") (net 4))
 (segment (start 103.39868 70.7) (end 104.7 70.7) (width 1) (layer "B.Cu") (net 4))
 (segment (start 94.9 83.1) (end 94.9 72.1) (width 1) (layer "B.Cu") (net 4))
 (segment (start 102.52 69) (end 102.52 69.82132) (width 1) (layer "B.Cu") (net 4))
 (segment (start 102.52 69.82132) (end 103.39868 70.7) (width 1) (layer "B.Cu") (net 4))
 (segment (start 82.5 82.5) (end 84.1 80.9) (width 1) (layer "F.Cu") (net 5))
 (segment (start 82.25 99.25) (end 84.6 101.6) (width 1) (layer "F.Cu") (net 5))
 (segment (start 84.1 80.9) (end 86 80.9) (width 1) (layer "F.Cu") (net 5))
 (segment (start 100 73.54) (end 93 73.54) (width 1) (layer "F.Cu") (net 5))
 (segment (start 84.6 101.6) (end 86.5 101.6) (width 1) (layer "F.Cu") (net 5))
 (via (at 93 73.54) (size 2) (drill 1) (layers "F.Cu" "B.Cu") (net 5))
 (via (at 82.5 82.5) (size 2) (drill 1) (layers "F.Cu" "B.Cu") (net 5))
 (via (at 82.25 99.25) (size 2) (drill 1) (layers "F.Cu" "B.Cu") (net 5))
 (segment (start 82.5 82.5) (end 82.5 74.5) (width 1) (layer "B.Cu") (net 5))
 (segment (start 81.75 99.25) (end 80.25 97.75) (width 1) (layer "B.Cu") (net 5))
 (segment (start 83.46 73.54) (end 93 73.54) (width 1) (layer "B.Cu") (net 5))
 (segment (start 82.5 74.5) (end 83.46 73.54) (width 1) (layer "B.Cu") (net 5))
 (segment (start 82.25 99.25) (end 81.75 99.25) (width 1) (layer "B.Cu") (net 5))
 (segment (start 80.25 84.75) (end 82.5 82.5) (width 1) (layer "B.Cu") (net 5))
 (segment (start 80.25 97.75) (end 80.25 84.75) (width 1) (layer "B.Cu") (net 5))
 (segment (start 93.08 52.42) (end 93.08 45.5) (width 1) (layer "F.Cu") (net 30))
 (segment (start 93.8 85.3) (end 93 85.3) (width 1) (layer "F.Cu") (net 30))
 (segment (start 93 52.5) (end 93.08 52.42) (width 1) (layer "F.Cu") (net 30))
 (segment (start 108.5 88.5) (end 97 88.5) (width 1) (layer "F.Cu") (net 30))
 (segment (start 97 88.5) (end 93.8 85.3) (width 1) (layer "F.Cu") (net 30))
 (via (at 108.5 88.5) (size 2) (drill 1) (layers "F.Cu" "B.Cu") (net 30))
 (via (at 93 52.5) (size 2) (drill 1) (layers "F.Cu" "B.Cu") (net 30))
 (segment (start 111.75 67.75) (end 111.75 88.5) (width 1) (layer "B.Cu") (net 30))
 (segment (start 111.75 88.5) (end 108.5 88.5) (width 1) (layer "B.Cu") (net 30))
 (segment (start 96.5 52.5) (end 111.75 67.75) (width 1) (layer "B.Cu") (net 30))
 (segment (start 93 52.5) (end 96.5 52.5) (width 1) (layer "B.Cu") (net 30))
 (segment (start 90.54 49.04) (end 90.54 45.5) (width 1) (layer "F.Cu") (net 29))
 (segment (start 91 49.5) (end 90.54 49.04) (width 1) (layer "F.Cu") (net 29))
 (segment (start 95 109) (end 96 109) (width 1) (layer "F.Cu") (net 29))
 (segment (start 92.2 103.8) (end 92 104) (width 1) (layer "F.Cu") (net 29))
 (segment (start 92 106) (end 95 109) (width 1) (layer "F.Cu") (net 29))
 (segment (start 93.5 103.8) (end 92.2 103.8) (width 1) (layer "F.Cu") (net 29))
 (segment (start 92 104) (end 92 106) (width 1) (layer "F.Cu") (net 29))
 (via (at 96 109) (size 2) (drill 1) (layers "F.Cu" "B.Cu") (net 29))
 (via (at 91 49.5) (size 2) (drill 1) (layers "F.Cu" "B.Cu") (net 29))
 (segment (start 107.5 109) (end 96 109) (width 1) (layer "B.Cu") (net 29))
 (segment (start 91 49.5) (end 96 49.5) (width 1) (layer "B.Cu") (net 29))
 (segment (start 114 67.5) (end 114 102.5) (width 1) (layer "B.Cu") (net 29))
 (segment (start 114 102.5) (end 107.5 109) (width 1) (layer "B.Cu") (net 29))
 (segment (start 96 49.5) (end 114 67.5) (width 1) (layer "B.Cu") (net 29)))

